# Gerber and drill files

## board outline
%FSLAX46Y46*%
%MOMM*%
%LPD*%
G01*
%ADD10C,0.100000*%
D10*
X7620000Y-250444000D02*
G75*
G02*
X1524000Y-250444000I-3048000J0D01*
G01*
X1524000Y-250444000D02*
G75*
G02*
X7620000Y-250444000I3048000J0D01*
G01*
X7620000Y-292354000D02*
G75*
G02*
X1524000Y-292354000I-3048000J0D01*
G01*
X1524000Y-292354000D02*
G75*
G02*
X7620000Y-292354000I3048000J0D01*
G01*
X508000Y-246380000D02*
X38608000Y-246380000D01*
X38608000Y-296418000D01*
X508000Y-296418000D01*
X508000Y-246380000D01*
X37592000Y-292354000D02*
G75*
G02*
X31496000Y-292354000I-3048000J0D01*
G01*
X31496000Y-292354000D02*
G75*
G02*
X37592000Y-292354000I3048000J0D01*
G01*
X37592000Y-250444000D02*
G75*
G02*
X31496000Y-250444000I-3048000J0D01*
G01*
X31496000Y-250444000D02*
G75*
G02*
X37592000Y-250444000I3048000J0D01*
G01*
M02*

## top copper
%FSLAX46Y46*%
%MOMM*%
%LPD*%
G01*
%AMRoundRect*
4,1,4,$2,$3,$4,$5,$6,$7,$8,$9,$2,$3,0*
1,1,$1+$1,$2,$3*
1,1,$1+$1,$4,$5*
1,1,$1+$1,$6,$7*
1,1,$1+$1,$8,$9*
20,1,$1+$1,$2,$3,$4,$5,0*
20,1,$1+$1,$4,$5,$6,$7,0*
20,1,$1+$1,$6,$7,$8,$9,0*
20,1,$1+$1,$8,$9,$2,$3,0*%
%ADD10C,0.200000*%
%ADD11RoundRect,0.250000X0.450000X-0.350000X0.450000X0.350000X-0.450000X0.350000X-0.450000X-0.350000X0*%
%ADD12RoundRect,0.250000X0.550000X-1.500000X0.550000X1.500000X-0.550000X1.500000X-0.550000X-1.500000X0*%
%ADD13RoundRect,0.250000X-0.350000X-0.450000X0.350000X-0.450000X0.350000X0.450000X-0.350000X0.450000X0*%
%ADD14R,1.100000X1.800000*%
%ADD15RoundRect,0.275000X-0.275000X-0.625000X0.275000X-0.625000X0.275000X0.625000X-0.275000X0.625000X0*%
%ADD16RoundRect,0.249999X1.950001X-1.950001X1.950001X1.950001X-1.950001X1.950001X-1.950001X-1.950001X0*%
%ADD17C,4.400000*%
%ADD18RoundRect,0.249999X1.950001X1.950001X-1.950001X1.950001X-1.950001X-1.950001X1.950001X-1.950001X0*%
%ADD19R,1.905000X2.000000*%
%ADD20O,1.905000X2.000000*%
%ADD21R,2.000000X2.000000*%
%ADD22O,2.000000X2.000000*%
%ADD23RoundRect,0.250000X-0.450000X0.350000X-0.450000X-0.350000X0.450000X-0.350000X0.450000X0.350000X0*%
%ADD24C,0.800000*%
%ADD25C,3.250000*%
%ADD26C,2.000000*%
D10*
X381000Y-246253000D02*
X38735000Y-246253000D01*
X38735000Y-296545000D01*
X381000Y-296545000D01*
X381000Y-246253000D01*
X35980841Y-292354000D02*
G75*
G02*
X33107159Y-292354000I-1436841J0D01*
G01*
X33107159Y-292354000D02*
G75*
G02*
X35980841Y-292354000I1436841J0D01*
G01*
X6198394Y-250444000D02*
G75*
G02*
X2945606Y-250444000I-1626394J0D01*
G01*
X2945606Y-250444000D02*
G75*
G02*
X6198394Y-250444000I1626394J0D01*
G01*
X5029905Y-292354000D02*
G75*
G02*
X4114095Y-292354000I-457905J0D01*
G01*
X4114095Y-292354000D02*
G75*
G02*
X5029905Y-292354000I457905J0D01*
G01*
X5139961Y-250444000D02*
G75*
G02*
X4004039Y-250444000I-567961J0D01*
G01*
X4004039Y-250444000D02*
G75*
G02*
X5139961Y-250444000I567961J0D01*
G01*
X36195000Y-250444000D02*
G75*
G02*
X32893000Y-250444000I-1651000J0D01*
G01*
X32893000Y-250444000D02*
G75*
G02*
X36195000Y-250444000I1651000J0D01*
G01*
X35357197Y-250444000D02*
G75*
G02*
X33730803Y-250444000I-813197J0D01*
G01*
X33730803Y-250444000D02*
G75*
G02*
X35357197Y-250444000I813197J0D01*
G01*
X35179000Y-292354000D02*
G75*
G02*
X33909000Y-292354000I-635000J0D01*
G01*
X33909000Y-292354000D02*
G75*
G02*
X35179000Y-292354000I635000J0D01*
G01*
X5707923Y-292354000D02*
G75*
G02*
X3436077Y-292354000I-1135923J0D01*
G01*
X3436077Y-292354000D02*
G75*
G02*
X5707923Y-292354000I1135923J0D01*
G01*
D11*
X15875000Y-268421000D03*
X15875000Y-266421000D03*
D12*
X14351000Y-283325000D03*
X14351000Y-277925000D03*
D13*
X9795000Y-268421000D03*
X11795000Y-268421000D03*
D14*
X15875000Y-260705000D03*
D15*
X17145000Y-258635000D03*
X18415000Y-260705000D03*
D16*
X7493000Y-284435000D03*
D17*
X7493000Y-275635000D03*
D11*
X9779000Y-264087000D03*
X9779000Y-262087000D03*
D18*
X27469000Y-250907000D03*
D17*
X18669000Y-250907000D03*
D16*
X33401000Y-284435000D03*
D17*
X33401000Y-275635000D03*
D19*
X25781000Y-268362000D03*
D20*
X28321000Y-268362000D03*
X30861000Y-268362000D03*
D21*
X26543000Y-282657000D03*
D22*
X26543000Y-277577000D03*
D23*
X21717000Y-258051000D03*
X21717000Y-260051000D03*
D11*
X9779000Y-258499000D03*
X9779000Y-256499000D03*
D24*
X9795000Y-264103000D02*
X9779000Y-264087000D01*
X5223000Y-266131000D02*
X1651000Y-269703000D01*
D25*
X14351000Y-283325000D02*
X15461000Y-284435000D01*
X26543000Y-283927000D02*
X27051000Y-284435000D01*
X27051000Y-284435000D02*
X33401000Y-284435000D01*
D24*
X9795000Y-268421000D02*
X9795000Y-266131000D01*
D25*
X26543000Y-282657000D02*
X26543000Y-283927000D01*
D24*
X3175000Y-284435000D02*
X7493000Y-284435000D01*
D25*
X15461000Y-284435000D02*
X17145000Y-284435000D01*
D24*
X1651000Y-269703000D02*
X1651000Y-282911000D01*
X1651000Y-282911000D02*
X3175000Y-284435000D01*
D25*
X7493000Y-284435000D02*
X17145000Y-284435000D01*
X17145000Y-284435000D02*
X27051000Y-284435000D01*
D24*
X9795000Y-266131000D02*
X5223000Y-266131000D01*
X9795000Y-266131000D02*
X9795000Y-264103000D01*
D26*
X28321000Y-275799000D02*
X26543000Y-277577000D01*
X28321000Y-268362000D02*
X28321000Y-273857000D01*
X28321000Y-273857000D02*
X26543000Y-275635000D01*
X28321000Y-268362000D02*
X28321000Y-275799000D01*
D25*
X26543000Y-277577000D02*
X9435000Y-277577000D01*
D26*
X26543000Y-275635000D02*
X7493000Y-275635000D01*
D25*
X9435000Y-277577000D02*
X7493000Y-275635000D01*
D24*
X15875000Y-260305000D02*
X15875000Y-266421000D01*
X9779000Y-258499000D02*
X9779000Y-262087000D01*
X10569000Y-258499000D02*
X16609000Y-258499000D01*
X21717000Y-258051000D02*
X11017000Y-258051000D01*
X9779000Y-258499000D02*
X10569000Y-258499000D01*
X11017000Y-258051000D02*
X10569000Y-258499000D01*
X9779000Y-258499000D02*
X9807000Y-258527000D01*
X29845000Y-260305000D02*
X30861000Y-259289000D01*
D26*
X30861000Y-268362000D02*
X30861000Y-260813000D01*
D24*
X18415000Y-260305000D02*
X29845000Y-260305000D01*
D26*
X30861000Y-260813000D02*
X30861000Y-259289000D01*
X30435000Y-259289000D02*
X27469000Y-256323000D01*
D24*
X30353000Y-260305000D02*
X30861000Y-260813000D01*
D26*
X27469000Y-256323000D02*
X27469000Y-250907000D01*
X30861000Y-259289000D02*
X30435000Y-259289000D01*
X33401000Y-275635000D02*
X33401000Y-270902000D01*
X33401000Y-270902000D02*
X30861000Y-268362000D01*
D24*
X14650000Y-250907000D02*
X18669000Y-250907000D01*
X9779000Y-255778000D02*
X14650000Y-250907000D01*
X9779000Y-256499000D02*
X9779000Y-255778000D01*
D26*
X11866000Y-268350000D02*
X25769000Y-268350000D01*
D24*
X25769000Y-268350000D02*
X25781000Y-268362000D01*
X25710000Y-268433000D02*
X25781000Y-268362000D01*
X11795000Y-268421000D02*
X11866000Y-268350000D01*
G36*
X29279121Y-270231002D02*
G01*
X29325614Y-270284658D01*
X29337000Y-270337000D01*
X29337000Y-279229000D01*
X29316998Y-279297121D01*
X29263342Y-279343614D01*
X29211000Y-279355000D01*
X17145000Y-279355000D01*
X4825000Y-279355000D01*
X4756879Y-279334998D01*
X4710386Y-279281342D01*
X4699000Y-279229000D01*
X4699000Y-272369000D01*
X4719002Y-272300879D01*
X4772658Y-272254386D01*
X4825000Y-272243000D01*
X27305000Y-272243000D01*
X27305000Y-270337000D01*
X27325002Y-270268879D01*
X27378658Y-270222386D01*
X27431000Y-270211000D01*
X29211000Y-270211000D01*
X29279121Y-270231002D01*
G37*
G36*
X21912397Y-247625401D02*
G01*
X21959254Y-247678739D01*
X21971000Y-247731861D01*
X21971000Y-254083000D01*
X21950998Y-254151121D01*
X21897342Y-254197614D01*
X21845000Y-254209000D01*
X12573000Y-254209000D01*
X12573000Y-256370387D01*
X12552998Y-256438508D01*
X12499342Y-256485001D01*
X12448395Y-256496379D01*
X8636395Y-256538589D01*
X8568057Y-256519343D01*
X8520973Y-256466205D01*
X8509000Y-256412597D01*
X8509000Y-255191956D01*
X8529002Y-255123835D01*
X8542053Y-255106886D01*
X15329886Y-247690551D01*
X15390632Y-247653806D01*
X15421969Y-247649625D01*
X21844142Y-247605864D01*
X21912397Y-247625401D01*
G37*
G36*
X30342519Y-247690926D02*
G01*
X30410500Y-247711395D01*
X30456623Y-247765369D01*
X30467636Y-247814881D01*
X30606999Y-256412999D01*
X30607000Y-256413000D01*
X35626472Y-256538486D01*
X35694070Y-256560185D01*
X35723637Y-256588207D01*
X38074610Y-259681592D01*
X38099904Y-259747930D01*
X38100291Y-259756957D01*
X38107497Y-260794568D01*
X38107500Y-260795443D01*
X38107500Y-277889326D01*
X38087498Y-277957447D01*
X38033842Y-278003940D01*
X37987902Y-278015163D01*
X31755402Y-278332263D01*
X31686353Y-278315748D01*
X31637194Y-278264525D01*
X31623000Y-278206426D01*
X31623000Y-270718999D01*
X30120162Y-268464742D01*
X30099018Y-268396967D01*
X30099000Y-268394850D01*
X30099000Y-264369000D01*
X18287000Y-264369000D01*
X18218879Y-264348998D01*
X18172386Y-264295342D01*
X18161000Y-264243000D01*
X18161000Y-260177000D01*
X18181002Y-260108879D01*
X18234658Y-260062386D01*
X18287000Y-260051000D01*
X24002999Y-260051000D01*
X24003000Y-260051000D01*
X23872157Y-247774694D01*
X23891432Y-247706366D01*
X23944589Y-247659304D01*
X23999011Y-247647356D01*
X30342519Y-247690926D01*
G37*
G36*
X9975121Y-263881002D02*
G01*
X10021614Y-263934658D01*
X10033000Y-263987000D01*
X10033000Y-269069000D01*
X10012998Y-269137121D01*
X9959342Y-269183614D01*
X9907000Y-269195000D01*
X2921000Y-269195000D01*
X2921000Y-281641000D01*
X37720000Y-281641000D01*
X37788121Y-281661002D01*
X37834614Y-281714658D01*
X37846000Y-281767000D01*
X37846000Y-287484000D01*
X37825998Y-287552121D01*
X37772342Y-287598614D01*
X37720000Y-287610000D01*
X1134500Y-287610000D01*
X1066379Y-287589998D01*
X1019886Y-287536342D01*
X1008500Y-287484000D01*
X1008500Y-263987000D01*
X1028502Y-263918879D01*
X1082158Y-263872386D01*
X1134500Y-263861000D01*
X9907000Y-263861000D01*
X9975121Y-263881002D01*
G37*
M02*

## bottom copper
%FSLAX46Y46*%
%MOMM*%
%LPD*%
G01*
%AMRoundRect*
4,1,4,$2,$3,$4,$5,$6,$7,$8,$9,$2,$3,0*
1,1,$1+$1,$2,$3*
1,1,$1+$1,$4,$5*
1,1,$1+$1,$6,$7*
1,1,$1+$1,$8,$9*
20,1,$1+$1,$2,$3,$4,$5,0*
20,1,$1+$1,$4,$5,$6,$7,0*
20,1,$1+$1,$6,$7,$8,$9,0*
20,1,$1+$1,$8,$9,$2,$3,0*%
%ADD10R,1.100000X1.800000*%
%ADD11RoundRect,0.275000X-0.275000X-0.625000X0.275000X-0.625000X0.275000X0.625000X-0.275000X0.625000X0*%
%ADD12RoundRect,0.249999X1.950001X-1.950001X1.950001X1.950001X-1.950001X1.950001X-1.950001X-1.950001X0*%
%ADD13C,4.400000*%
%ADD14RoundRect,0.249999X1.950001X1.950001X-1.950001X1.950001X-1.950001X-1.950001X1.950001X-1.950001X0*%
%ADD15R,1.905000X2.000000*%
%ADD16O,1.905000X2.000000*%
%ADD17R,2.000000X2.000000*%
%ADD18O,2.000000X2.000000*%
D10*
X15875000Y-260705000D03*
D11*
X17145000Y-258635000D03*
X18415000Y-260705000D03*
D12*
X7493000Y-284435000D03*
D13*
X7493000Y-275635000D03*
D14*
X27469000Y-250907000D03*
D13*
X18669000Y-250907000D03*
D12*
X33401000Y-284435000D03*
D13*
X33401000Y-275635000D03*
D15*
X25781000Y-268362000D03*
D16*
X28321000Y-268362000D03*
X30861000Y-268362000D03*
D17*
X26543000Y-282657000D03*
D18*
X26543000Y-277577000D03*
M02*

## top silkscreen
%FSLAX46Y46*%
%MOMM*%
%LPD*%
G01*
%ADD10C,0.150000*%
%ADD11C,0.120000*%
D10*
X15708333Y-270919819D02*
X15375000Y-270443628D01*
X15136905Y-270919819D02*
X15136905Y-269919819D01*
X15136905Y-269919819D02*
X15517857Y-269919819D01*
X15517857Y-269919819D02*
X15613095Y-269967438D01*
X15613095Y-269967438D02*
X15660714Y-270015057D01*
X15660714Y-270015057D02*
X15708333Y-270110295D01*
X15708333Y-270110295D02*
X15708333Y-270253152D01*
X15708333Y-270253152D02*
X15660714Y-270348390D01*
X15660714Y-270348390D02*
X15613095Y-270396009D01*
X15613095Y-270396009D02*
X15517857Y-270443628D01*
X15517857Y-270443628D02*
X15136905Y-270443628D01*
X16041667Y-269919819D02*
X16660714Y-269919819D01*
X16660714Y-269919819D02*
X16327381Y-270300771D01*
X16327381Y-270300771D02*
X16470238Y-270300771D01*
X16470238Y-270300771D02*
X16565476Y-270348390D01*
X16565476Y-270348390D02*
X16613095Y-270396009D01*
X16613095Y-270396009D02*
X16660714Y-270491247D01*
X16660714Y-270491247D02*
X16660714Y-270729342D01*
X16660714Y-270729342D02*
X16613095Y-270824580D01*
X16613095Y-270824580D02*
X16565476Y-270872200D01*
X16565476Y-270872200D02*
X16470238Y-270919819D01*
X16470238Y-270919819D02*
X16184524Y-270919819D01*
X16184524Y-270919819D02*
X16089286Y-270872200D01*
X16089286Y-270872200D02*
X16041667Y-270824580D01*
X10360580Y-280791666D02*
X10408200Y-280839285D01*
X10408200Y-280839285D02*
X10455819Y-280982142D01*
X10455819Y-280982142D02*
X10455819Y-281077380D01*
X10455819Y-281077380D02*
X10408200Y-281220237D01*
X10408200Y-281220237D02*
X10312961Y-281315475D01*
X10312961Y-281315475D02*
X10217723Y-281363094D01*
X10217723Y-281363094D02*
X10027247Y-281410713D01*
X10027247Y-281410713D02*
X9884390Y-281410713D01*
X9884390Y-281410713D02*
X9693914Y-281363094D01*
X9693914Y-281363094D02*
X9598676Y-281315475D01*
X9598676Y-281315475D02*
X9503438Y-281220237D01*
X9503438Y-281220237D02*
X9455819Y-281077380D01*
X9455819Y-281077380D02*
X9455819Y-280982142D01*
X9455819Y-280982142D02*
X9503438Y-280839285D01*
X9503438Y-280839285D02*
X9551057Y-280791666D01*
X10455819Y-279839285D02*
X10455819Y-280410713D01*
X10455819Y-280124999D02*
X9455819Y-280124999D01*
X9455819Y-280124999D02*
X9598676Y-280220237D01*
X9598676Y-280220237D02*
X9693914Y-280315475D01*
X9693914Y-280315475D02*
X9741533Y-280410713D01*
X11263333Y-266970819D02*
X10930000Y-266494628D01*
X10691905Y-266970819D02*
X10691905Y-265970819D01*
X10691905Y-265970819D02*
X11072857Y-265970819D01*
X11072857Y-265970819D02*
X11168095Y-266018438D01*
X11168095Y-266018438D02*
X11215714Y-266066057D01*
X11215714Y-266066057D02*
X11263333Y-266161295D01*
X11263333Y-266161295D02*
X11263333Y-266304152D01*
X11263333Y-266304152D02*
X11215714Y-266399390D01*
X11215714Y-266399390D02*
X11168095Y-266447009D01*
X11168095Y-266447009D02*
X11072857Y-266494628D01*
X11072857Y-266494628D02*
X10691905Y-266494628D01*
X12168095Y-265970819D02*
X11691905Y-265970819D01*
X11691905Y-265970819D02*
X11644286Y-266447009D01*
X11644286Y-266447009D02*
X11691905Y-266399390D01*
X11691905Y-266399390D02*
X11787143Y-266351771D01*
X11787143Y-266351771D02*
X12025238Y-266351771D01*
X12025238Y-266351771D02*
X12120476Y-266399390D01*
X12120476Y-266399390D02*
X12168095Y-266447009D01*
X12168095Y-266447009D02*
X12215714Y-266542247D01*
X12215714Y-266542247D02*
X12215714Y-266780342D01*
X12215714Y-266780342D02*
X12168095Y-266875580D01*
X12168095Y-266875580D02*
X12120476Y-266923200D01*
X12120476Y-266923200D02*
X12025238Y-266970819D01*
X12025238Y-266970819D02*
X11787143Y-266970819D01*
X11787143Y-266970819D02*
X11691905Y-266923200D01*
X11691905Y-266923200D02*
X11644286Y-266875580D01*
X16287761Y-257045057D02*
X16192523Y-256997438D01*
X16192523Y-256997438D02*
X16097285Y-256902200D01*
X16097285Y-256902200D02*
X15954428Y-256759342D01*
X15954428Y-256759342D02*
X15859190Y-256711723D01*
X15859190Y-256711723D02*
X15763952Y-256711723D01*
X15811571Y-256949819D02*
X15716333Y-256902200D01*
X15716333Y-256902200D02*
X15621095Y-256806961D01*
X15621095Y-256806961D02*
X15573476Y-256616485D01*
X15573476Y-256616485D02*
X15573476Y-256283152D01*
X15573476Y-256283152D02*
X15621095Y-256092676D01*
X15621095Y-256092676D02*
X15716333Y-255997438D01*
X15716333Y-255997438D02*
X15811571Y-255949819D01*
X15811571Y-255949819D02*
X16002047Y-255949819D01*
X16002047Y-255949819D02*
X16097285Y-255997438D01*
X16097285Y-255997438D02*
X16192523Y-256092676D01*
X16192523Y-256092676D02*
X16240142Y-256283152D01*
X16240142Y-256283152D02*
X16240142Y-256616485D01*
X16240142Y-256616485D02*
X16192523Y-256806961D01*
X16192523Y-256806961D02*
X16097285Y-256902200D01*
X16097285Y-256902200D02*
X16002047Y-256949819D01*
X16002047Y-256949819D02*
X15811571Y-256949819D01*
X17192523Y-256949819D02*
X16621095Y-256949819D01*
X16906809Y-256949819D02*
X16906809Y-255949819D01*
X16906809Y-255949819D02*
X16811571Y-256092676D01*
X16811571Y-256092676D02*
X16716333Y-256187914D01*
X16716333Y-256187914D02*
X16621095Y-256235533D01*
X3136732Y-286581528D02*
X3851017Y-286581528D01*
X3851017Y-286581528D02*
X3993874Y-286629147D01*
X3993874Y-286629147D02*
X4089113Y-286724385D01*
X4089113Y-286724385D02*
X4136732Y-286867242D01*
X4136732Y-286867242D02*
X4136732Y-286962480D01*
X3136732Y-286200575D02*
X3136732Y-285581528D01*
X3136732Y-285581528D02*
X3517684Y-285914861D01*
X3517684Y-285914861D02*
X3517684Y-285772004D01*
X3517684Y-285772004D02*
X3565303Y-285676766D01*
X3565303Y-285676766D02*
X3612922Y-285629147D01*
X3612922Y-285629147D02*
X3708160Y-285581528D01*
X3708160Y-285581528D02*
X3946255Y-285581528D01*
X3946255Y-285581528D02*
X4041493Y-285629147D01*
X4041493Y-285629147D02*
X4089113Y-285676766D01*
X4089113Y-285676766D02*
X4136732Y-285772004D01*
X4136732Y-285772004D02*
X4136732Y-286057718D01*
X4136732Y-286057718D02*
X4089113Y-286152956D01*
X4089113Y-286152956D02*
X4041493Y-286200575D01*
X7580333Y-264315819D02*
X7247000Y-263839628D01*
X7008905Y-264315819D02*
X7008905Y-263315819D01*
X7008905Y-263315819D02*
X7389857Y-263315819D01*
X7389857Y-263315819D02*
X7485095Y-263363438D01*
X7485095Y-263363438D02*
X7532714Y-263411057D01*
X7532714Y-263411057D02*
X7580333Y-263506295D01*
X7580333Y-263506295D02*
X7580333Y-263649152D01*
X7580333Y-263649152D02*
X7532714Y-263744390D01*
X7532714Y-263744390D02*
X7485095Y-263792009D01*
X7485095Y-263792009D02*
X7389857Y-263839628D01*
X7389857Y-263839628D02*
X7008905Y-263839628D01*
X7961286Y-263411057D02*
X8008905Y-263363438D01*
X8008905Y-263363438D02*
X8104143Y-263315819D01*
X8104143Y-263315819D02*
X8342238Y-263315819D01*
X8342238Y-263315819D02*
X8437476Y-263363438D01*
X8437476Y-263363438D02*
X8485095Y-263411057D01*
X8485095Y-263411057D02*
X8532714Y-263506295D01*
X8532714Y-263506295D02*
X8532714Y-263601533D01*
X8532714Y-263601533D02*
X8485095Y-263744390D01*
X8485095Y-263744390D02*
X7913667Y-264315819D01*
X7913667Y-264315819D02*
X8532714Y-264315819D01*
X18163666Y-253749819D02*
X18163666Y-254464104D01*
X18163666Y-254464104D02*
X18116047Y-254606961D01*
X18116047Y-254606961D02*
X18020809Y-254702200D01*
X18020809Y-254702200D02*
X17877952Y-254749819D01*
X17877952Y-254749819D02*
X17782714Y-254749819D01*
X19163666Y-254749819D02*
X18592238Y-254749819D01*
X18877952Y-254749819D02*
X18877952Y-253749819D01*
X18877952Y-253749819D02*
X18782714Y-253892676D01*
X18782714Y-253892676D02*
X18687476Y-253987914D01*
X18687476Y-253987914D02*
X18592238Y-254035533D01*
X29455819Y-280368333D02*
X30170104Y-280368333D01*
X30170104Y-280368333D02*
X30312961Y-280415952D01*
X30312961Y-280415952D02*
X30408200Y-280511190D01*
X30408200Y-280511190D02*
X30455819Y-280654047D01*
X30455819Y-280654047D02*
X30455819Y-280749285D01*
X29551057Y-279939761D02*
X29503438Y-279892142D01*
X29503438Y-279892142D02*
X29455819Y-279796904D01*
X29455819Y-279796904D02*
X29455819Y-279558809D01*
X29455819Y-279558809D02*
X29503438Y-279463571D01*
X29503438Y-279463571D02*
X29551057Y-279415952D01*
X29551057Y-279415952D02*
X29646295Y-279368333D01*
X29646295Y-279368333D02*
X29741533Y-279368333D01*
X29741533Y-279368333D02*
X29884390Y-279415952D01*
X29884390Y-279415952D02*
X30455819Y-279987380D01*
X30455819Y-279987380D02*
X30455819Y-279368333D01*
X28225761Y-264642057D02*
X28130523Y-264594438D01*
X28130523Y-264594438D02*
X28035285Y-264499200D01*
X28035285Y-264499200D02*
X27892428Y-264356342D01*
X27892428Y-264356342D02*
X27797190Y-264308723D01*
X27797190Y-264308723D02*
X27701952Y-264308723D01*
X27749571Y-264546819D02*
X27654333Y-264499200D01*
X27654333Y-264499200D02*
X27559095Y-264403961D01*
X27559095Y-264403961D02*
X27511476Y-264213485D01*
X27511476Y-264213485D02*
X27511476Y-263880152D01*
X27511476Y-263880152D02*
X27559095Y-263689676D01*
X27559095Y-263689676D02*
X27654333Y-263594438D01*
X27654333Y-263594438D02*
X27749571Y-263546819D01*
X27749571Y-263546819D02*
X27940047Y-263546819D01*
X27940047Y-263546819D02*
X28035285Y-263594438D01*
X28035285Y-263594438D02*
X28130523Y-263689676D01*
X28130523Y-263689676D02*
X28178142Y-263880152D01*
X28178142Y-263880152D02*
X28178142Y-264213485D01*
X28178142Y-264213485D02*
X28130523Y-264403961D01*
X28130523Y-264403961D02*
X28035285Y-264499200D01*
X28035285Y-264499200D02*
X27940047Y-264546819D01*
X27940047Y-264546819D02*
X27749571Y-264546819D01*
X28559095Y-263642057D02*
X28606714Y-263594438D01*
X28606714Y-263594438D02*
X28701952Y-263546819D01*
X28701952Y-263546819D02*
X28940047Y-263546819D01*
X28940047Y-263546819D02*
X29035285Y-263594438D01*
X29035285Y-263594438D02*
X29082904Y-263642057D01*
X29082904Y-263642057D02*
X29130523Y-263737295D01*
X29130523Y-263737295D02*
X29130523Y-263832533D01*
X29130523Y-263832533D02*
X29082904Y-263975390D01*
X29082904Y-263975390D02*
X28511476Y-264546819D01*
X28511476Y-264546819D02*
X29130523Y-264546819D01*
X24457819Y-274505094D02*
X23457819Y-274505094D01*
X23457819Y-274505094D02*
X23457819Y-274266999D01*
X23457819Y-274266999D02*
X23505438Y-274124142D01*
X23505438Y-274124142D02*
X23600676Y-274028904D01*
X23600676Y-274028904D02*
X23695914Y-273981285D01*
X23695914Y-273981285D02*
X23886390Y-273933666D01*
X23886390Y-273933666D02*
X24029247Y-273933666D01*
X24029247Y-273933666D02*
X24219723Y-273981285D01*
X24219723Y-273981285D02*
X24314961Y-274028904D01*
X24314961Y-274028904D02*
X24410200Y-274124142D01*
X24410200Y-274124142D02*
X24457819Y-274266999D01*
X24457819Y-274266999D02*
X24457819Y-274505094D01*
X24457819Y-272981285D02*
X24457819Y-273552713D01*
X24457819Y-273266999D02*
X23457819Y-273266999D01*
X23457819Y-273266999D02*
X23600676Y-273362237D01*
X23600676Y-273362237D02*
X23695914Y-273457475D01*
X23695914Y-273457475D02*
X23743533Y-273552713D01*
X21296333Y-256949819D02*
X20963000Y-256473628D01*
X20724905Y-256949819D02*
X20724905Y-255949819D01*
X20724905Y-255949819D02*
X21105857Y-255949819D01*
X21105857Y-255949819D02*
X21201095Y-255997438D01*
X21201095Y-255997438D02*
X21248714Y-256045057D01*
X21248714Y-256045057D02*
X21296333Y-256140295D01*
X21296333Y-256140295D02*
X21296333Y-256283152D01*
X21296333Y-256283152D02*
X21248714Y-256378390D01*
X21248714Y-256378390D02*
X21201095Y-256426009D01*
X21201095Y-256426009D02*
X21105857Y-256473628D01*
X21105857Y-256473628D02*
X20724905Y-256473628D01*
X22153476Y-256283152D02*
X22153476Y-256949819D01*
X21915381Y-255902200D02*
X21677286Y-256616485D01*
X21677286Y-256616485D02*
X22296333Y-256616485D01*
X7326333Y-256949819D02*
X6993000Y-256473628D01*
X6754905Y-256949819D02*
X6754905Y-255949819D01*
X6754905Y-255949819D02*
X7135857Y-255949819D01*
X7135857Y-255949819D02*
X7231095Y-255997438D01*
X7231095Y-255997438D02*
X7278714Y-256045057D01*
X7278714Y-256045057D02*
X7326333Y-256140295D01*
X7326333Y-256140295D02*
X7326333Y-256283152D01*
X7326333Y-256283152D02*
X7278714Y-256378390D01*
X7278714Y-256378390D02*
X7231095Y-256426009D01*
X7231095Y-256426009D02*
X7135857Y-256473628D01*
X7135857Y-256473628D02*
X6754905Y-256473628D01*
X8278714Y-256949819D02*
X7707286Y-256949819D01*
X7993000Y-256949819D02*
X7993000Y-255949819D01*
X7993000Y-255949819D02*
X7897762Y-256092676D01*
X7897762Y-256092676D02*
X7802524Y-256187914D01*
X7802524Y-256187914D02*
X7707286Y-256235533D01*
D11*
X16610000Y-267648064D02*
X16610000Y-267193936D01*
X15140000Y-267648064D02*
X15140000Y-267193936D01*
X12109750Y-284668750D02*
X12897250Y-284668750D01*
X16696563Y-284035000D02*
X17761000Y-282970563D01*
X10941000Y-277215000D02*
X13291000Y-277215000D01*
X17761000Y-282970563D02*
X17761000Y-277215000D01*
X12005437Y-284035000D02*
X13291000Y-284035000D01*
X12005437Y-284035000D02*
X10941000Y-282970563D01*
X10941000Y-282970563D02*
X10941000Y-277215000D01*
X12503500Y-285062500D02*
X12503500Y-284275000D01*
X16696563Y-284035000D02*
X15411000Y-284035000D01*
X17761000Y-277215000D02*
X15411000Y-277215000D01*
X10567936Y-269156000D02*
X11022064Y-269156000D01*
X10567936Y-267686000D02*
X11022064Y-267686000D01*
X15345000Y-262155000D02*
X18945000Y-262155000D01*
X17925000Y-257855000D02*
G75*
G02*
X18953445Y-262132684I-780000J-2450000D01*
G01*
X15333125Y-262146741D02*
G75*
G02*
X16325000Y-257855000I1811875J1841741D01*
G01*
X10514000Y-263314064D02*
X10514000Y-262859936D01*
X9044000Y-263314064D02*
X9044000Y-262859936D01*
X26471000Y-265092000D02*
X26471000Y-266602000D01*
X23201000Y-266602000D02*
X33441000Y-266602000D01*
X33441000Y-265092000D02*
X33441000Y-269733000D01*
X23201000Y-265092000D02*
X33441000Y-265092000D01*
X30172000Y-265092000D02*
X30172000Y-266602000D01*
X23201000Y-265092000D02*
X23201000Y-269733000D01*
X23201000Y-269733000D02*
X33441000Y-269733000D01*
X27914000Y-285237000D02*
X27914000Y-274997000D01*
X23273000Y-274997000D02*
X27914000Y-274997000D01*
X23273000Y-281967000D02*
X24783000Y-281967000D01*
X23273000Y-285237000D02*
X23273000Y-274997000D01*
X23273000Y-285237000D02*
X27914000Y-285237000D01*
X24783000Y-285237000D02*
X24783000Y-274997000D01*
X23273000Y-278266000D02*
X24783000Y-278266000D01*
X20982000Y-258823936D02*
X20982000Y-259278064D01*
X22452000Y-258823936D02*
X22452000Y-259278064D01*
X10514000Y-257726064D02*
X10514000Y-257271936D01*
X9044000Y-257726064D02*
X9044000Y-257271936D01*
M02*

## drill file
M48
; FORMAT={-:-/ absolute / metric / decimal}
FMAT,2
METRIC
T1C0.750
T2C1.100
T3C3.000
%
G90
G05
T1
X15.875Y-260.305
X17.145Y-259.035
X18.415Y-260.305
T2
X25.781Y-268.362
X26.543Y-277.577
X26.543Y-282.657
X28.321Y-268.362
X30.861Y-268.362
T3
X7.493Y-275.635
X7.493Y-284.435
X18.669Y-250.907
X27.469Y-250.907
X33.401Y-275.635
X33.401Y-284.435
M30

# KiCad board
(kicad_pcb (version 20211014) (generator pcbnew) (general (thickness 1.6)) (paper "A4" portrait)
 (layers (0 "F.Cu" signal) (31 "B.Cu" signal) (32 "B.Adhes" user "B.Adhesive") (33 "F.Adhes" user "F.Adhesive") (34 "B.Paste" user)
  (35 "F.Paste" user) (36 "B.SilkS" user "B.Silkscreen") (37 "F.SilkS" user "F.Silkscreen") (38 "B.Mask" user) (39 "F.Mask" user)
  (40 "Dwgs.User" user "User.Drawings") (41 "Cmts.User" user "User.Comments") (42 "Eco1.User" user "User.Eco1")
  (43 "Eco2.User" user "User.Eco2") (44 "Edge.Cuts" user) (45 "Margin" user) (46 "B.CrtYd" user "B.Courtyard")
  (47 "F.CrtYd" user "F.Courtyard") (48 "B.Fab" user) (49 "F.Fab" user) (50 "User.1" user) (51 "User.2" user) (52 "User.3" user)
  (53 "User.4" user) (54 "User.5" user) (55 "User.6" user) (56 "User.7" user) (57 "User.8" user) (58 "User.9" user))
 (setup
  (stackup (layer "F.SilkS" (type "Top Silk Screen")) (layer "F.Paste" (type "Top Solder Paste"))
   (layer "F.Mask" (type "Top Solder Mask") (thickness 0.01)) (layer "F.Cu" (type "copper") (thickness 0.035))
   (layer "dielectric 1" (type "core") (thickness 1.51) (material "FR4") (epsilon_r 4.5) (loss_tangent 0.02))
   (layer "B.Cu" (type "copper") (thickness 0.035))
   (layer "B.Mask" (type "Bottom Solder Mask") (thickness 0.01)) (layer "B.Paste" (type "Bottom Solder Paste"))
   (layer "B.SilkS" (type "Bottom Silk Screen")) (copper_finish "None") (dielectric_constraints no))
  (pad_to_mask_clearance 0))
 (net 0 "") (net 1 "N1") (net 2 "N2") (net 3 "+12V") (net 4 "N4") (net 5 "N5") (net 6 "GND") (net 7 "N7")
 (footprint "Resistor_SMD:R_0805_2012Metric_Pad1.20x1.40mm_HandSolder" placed (layer "F.Cu") (at 15.875 267.421 90)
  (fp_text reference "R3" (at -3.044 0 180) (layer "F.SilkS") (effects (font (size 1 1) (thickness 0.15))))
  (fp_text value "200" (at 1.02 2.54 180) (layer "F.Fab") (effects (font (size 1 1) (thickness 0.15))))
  (fp_line (start -0.227064 0.735) (end 0.227064 0.735) (layer "F.SilkS") (width 0.12))
  (fp_line (start -0.227064 -0.735) (end 0.227064 -0.735) (layer "F.SilkS") (width 0.12))
  (pad "1" smd roundrect (at -1 0 90) (size 1.2 1.4) (layers "F.Cu" "F.Paste" "F.Mask") (roundrect_rratio 0.2083333333) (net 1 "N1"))
  (pad "2" smd roundrect (at 1 0 90) (size 1.2 1.4) (layers "F.Cu" "F.Paste" "F.Mask") (roundrect_rratio 0.2083333333) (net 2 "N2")))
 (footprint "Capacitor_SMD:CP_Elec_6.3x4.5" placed (layer "F.Cu") (at 14.351 280.625 90)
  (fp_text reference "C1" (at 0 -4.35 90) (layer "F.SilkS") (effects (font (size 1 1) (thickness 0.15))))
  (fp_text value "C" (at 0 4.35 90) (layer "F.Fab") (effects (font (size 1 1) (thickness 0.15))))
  (fp_line (start -4.04375 -2.24125) (end -4.04375 -1.45375) (layer "F.SilkS") (width 0.12))
  (fp_line (start -3.41 2.345563) (end -2.345563 3.41) (layer "F.SilkS") (width 0.12))
  (fp_line (start 3.41 -3.41) (end 3.41 -1.06) (layer "F.SilkS") (width 0.12))
  (fp_line (start -2.345563 3.41) (end 3.41 3.41) (layer "F.SilkS") (width 0.12))
  (fp_line (start -3.41 -2.345563) (end -3.41 -1.06) (layer "F.SilkS") (width 0.12))
  (fp_line (start -3.41 -2.345563) (end -2.345563 -3.41) (layer "F.SilkS") (width 0.12))
  (fp_line (start -2.345563 -3.41) (end 3.41 -3.41) (layer "F.SilkS") (width 0.12))
  (fp_line (start -4.4375 -1.8475) (end -3.65 -1.8475) (layer "F.SilkS") (width 0.12))
  (fp_line (start -3.41 2.345563) (end -3.41 1.06) (layer "F.SilkS") (width 0.12))
  (fp_line (start 3.41 3.41) (end 3.41 1.06) (layer "F.SilkS") (width 0.12))
  (pad "1" smd roundrect (at -2.7 0 90) (size 3.5 1.6) (layers "F.Cu" "F.Paste" "F.Mask") (roundrect_rratio 0.15625) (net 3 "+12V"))
  (pad "2" smd roundrect (at 2.7 0 90) (size 3.5 1.6) (layers "F.Cu" "F.Paste" "F.Mask") (roundrect_rratio 0.15625) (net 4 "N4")))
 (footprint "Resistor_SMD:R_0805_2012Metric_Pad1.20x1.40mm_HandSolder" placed (layer "F.Cu") (at 10.795 268.421)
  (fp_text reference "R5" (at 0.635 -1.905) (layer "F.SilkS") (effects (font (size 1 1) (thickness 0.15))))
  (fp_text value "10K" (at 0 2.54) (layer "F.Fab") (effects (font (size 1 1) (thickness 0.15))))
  (fp_line (start -0.227064 0.735) (end 0.227064 0.735) (layer "F.SilkS") (width 0.12))
  (fp_line (start -0.227064 -0.735) (end 0.227064 -0.735) (layer "F.SilkS") (width 0.12))
  (pad "1" smd roundrect (at -1 0) (size 1.2 1.4) (layers "F.Cu" "F.Paste" "F.Mask") (roundrect_rratio 0.2083333333) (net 3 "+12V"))
  (pad "2" smd roundrect (at 1 0) (size 1.2 1.4) (layers "F.Cu" "F.Paste" "F.Mask") (roundrect_rratio 0.2083333333) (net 1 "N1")))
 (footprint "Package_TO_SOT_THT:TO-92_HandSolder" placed (layer "F.Cu") (at 15.875 260.305)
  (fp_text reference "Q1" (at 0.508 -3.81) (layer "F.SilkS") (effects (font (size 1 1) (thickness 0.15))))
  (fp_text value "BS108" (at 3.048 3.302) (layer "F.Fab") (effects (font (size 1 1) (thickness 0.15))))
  (fp_line (start -0.53 1.85) (end 3.07 1.85) (layer "F.SilkS") (width 0.12))
  (fp_arc (start 2.05 -2.45) (mid 3.769931 -0.601036) (end 3.078445 1.827684) (layer "F.SilkS") (width 0.12))
  (fp_arc (start -0.541875 1.841741) (mid -1.247231 -0.581764) (end 0.45 -2.45) (layer "F.SilkS") (width 0.12))
  (pad "1" thru_hole rect (at 0 0) (size 1.1 1.8) (drill 0.75 (offset 0 0.4)) (layers *.Cu *.Mask) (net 2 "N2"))
  (pad "2" thru_hole roundrect (at 1.27 -1.27) (size 1.1 1.8) (drill 0.75 (offset 0 -0.4)) (layers *.Cu *.Mask) (roundrect_rratio 0.25)
   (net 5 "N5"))
  (pad "3" thru_hole roundrect (at 2.54 0) (size 1.1 1.8) (drill 0.75 (offset 0 0.4)) (layers *.Cu *.Mask) (roundrect_rratio 0.25)
   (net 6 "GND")))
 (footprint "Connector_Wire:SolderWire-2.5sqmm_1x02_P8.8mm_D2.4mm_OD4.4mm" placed (layer "F.Cu") (at 7.493 284.435 90)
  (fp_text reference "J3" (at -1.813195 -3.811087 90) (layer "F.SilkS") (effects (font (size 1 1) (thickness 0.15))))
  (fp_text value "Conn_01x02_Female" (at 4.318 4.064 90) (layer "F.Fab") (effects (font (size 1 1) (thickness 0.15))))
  (pad "1" thru_hole roundrect (at 0 0 90) (size 4.4 4.4) (drill 3) (layers *.Cu *.Mask) (roundrect_rratio 0.05681795455) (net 3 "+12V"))
  (pad "2" thru_hole circle (at 8.8 0 90) (size 4.4 4.4) (drill 3) (layers *.Cu *.Mask) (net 4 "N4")))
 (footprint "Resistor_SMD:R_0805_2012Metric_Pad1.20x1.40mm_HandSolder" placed (layer "F.Cu") (at 9.779 263.087 90)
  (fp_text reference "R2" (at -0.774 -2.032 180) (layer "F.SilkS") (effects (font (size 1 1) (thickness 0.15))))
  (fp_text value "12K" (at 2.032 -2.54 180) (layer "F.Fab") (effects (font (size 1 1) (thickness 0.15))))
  (fp_line (start -0.227064 0.735) (end 0.227064 0.735) (layer "F.SilkS") (width 0.12))
  (fp_line (start -0.227064 -0.735) (end 0.227064 -0.735) (layer "F.SilkS") (width 0.12))
  (pad "1" smd roundrect (at -1 0 90) (size 1.2 1.4) (layers "F.Cu" "F.Paste" "F.Mask") (roundrect_rratio 0.2083333333) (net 3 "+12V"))
  (pad "2" smd roundrect (at 1 0 90) (size 1.2 1.4) (layers "F.Cu" "F.Paste" "F.Mask") (roundrect_rratio 0.2083333333) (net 5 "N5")))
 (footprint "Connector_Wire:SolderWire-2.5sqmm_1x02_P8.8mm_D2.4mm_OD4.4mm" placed (layer "F.Cu") (at 27.469 250.907 180)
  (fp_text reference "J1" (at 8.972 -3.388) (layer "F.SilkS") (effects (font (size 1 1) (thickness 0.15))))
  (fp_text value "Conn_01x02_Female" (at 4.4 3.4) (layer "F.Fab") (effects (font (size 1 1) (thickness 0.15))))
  (pad "1" thru_hole roundrect (at 0 0 180) (size 4.4 4.4) (drill 3) (layers *.Cu *.Mask) (roundrect_rratio 0.05681795455) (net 6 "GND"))
  (pad "2" thru_hole circle (at 8.8 0 180) (size 4.4 4.4) (drill 3) (layers *.Cu *.Mask) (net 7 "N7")))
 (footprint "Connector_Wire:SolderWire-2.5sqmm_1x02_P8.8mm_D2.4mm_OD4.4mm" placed (layer "F.Cu") (at 33.401 284.435 90)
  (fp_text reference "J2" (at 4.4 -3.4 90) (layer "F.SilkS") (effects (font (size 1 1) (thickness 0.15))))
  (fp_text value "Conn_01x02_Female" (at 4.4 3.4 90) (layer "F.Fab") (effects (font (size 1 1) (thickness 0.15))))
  (pad "1" thru_hole roundrect (at 0 0 90) (size 4.4 4.4) (drill 3) (layers *.Cu *.Mask) (roundrect_rratio 0.05681795455) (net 3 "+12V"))
  (pad "2" thru_hole circle (at 8.8 0 90) (size 4.4 4.4) (drill 3) (layers *.Cu *.Mask) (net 6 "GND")))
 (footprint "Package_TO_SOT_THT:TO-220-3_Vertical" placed (layer "F.Cu") (at 25.781 268.362)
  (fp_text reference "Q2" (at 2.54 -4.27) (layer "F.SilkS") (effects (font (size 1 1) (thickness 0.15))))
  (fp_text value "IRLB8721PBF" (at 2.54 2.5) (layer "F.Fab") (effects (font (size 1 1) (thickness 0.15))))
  (fp_line (start 0.69 -3.27) (end 0.69 -1.76) (layer "F.SilkS") (width 0.12))
  (fp_line (start -2.58 -1.76) (end 7.66 -1.76) (layer "F.SilkS") (width 0.12))
  (fp_line (start 7.66 -3.27) (end 7.66 1.371) (layer "F.SilkS") (width 0.12))
  (fp_line (start -2.58 -3.27) (end 7.66 -3.27) (layer "F.SilkS") (width 0.12))
  (fp_line (start 4.391 -3.27) (end 4.391 -1.76) (layer "F.SilkS") (width 0.12))
  (fp_line (start -2.58 -3.27) (end -2.58 1.371) (layer "F.SilkS") (width 0.12))
  (fp_line (start -2.58 1.371) (end 7.66 1.371) (layer "F.SilkS") (width 0.12))
  (pad "1" thru_hole rect (at 0 0) (size 1.905 2) (drill 1.1) (layers *.Cu *.Mask) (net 1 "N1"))
  (pad "2" thru_hole oval (at 2.54 0) (size 1.905 2) (drill 1.1) (layers *.Cu *.Mask) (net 4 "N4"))
  (pad "3" thru_hole oval (at 5.08 0) (size 1.905 2) (drill 1.1) (layers *.Cu *.Mask) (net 6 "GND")))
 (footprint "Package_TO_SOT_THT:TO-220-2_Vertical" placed (layer "F.Cu") (at 26.543 282.657 90)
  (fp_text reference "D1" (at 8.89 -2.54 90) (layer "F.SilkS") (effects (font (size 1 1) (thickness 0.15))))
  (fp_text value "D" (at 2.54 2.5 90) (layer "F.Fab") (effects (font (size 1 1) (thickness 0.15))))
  (fp_line (start -2.58 1.371) (end 7.66 1.371) (layer "F.SilkS") (width 0.12))
  (fp_line (start 7.66 -3.27) (end 7.66 1.371) (layer "F.SilkS") (width 0.12))
  (fp_line (start 0.69 -3.27) (end 0.69 -1.76) (layer "F.SilkS") (width 0.12))
  (fp_line (start -2.58 -3.27) (end 7.66 -3.27) (layer "F.SilkS") (width 0.12))
  (fp_line (start -2.58 -3.27) (end -2.58 1.371) (layer "F.SilkS") (width 0.12))
  (fp_line (start -2.58 -1.76) (end 7.66 -1.76) (layer "F.SilkS") (width 0.12))
  (fp_line (start 4.391 -3.27) (end 4.391 -1.76) (layer "F.SilkS") (width 0.12))
  (pad "1" thru_hole rect (at 0 0 90) (size 2 2) (drill 1.1) (layers *.Cu *.Mask) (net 3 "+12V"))
  (pad "2" thru_hole oval (at 5.08 0 90) (size 2 2) (drill 1.1) (layers *.Cu *.Mask) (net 4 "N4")))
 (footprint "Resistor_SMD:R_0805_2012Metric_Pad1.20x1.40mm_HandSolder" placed (layer "F.Cu") (at 21.717 259.051 -90)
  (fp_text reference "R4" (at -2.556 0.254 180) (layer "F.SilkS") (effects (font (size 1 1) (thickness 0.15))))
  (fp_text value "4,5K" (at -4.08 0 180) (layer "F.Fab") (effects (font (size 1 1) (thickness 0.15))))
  (fp_line (start -0.227064 0.735) (end 0.227064 0.735) (layer "F.SilkS") (width 0.12))
  (fp_line (start -0.227064 -0.735) (end 0.227064 -0.735) (layer "F.SilkS") (width 0.12))
  (pad "1" smd roundrect (at -1 0 270) (size 1.2 1.4) (layers "F.Cu" "F.Paste" "F.Mask") (roundrect_rratio 0.2083333333) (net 5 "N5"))
  (pad "2" smd roundrect (at 1 0 270) (size 1.2 1.4) (layers "F.Cu" "F.Paste" "F.Mask") (roundrect_rratio 0.2083333333) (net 6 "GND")))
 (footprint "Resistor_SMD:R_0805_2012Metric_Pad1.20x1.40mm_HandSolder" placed (layer "F.Cu") (at 9.779 257.499 90)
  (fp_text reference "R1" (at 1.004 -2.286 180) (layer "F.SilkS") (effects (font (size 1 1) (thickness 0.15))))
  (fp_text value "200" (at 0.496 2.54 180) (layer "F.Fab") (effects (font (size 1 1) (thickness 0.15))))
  (fp_line (start -0.227064 0.735) (end 0.227064 0.735) (layer "F.SilkS") (width 0.12))
  (fp_line (start -0.227064 -0.735) (end 0.227064 -0.735) (layer "F.SilkS") (width 0.12))
  (pad "1" smd roundrect (at -1 0 90) (size 1.2 1.4) (layers "F.Cu" "F.Paste" "F.Mask") (roundrect_rratio 0.2083333333) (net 5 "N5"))
  (pad "2" smd roundrect (at 1 0 90) (size 1.2 1.4) (layers "F.Cu" "F.Paste" "F.Mask") (roundrect_rratio 0.2083333333) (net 7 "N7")))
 (gr_rect (start 38.735 246.253) (end 0.381 296.545) (layer "F.Cu") (width 0.2) (fill none))
 (gr_circle (center 34.544 292.354) (end 35.56 293.37) (layer "F.Cu") (width 0.2) (fill none))
 (gr_circle (center 4.572 250.444) (end 5.588 251.714) (layer "F.Cu") (width 0.2) (fill none))
 (gr_circle (center 4.572 292.354) (end 4.826 292.735) (layer "F.Cu") (width 0.2) (fill none))
 (gr_circle (center 4.572 250.444) (end 4.826 250.952) (layer "F.Cu") (width 0.2) (fill none))
 (gr_circle (center 34.544 250.444) (end 35.179 248.92) (layer "F.Cu") (width 0.2) (fill none))
 (gr_circle (center 34.544 250.444) (end 35.052 251.079) (layer "F.Cu") (width 0.2) (fill none))
 (gr_circle (center 34.544 292.354) (end 34.925 292.862) (layer "F.Cu") (width 0.2) (fill none))
 (gr_circle (center 4.572 292.354) (end 5.08 293.37) (layer "F.Cu") (width 0.2) (fill none))
 (gr_circle (center 4.572 250.444) (end 4.572 247.396) (layer "Edge.Cuts") (width 0.1) (fill none))
 (gr_circle (center 4.572 292.354) (end 1.524 292.354) (layer "Edge.Cuts") (width 0.1) (fill none))
 (gr_rect (start 0.508 246.38) (end 38.608 296.418) (layer "Edge.Cuts") (width 0.1) (fill none))
 (gr_circle (center 34.544 292.354) (end 34.544 295.402) (layer "Edge.Cuts") (width 0.1) (fill none))
 (gr_circle (center 34.544 250.444) (end 37.592 250.444) (layer "Edge.Cuts") (width 0.1) (fill none))
 (segment (start 9.795 264.103) (end 9.779 264.087) (width 0.8) (layer "F.Cu") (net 3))
 (segment (start 5.223 266.131) (end 1.651 269.703) (width 0.8) (layer "F.Cu") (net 3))
 (segment (start 14.351 283.325) (end 15.461 284.435) (width 3.25) (layer "F.Cu") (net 3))
 (segment (start 26.543 283.927) (end 27.051 284.435) (width 3.25) (layer "F.Cu") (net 3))
 (segment (start 27.051 284.435) (end 33.401 284.435) (width 3.25) (layer "F.Cu") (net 3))
 (segment (start 9.795 268.421) (end 9.795 266.131) (width 0.8) (layer "F.Cu") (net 3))
 (segment (start 26.543 282.657) (end 26.543 283.927) (width 3.25) (layer "F.Cu") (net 3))
 (segment (start 3.175 284.435) (end 7.493 284.435) (width 0.8) (layer "F.Cu") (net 3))
 (segment (start 15.461 284.435) (end 17.145 284.435) (width 3.25) (layer "F.Cu") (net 3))
 (segment (start 1.651 269.703) (end 1.651 282.911) (width 0.8) (layer "F.Cu") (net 3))
 (segment (start 1.651 282.911) (end 3.175 284.435) (width 0.8) (layer "F.Cu") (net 3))
 (segment (start 7.493 284.435) (end 17.145 284.435) (width 3.25) (layer "F.Cu") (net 3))
 (segment (start 17.145 284.435) (end 27.051 284.435) (width 3.25) (layer "F.Cu") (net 3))
 (segment (start 9.795 266.131) (end 5.223 266.131) (width 0.8) (layer "F.Cu") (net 3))
 (segment (start 9.795 266.131) (end 9.795 264.103) (width 0.8) (layer "F.Cu") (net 3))
 (segment (start 28.321 275.799) (end 26.543 277.577) (width 2) (layer "F.Cu") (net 4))
 (segment (start 28.321 268.362) (end 28.321 273.857) (width 2) (layer "F.Cu") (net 4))
 (segment (start 28.321 273.857) (end 26.543 275.635) (width 2) (layer "F.Cu") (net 4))
 (segment (start 28.321 268.362) (end 28.321 275.799) (width 2) (layer "F.Cu") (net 4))
 (segment (start 26.543 277.577) (end 9.435 277.577) (width 3.25) (layer "F.Cu") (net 4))
 (segment (start 26.543 275.635) (end 7.493 275.635) (width 2) (layer "F.Cu") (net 4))
 (segment (start 9.435 277.577) (end 7.493 275.635) (width 3.25) (layer "F.Cu") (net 4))
 (segment (start 15.875 260.305) (end 15.875 266.421) (width 0.8) (layer "F.Cu") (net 2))
 (segment (start 9.779 258.499) (end 9.779 262.087) (width 0.8) (layer "F.Cu") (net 5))
 (segment (start 10.569 258.499) (end 16.609 258.499) (width 0.8) (layer "F.Cu") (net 5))
 (segment (start 21.717 258.051) (end 11.017 258.051) (width 0.8) (layer "F.Cu") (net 5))
 (segment (start 9.779 258.499) (end 10.569 258.499) (width 0.8) (layer "F.Cu") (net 5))
 (segment (start 11.017 258.051) (end 10.569 258.499) (width 0.8) (layer "F.Cu") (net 5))
 (segment (start 9.779 258.499) (end 9.807 258.527) (width 0.8) (layer "F.Cu") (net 5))
 (segment (start 29.845 260.305) (end 30.861 259.289) (width 0.8) (layer "F.Cu") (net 6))
 (segment (start 30.861 268.362) (end 30.861 260.813) (width 2) (layer "F.Cu") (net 6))
 (segment (start 18.415 260.305) (end 29.845 260.305) (width 0.8) (layer "F.Cu") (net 6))
 (segment (start 30.861 260.813) (end 30.861 259.289) (width 2) (layer "F.Cu") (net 6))
 (segment (start 30.435 259.289) (end 27.469 256.323) (width 2) (layer "F.Cu") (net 6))
 (segment (start 30.353 260.305) (end 30.861 260.813) (width 0.8) (layer "F.Cu") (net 6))
 (segment (start 27.469 256.323) (end 27.469 250.907) (width 2) (layer "F.Cu") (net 6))
 (segment (start 30.861 259.289) (end 30.435 259.289) (width 2) (layer "F.Cu") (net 6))
 (segment (start 33.401 275.635) (end 33.401 270.902) (width 2) (layer "F.Cu") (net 6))
 (segment (start 33.401 270.902) (end 30.861 268.362) (width 2) (layer "F.Cu") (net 6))
 (segment (start 14.65 250.907) (end 18.669 250.907) (width 0.8) (layer "F.Cu") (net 7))
 (segment (start 9.779 255.778) (end 14.65 250.907) (width 0.8) (layer "F.Cu") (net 7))
 (segment (start 9.779 256.499) (end 9.779 255.778) (width 0.8) (layer "F.Cu") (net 7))
 (segment (start 11.866 268.35) (end 25.769 268.35) (width 2) (layer "F.Cu") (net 1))
 (segment (start 25.769 268.35) (end 25.781 268.362) (width 0.8) (layer "F.Cu") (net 1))
 (segment (start 25.71 268.433) (end 25.781 268.362) (width 0.8) (layer "F.Cu") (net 1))
 (segment (start 11.795 268.421) (end 11.866 268.35) (width 0.8) (layer "F.Cu") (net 1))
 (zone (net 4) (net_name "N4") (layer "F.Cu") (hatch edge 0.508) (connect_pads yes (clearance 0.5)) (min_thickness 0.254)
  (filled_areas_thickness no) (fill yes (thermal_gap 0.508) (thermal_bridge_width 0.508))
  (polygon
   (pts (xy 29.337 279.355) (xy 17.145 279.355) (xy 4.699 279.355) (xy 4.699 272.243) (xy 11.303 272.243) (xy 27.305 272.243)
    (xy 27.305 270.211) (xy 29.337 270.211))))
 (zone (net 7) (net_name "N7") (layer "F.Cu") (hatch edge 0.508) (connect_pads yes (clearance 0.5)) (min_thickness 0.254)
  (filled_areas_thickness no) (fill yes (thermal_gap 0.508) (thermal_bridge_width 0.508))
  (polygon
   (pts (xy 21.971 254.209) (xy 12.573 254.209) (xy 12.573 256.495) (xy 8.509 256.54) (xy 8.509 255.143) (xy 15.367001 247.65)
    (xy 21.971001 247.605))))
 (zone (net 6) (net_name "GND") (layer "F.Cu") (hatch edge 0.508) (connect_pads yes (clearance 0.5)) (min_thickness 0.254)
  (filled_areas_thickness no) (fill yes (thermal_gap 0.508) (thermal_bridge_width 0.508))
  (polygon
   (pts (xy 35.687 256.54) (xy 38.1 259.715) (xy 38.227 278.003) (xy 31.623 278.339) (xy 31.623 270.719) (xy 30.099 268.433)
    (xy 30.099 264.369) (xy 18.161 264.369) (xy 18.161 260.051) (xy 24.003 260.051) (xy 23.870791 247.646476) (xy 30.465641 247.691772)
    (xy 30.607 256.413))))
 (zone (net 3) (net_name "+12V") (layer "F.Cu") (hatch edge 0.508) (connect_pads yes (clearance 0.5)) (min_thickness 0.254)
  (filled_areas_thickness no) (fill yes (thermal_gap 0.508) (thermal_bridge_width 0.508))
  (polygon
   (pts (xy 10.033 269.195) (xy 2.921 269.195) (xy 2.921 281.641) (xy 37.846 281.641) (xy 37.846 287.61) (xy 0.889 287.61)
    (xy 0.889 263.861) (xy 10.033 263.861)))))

